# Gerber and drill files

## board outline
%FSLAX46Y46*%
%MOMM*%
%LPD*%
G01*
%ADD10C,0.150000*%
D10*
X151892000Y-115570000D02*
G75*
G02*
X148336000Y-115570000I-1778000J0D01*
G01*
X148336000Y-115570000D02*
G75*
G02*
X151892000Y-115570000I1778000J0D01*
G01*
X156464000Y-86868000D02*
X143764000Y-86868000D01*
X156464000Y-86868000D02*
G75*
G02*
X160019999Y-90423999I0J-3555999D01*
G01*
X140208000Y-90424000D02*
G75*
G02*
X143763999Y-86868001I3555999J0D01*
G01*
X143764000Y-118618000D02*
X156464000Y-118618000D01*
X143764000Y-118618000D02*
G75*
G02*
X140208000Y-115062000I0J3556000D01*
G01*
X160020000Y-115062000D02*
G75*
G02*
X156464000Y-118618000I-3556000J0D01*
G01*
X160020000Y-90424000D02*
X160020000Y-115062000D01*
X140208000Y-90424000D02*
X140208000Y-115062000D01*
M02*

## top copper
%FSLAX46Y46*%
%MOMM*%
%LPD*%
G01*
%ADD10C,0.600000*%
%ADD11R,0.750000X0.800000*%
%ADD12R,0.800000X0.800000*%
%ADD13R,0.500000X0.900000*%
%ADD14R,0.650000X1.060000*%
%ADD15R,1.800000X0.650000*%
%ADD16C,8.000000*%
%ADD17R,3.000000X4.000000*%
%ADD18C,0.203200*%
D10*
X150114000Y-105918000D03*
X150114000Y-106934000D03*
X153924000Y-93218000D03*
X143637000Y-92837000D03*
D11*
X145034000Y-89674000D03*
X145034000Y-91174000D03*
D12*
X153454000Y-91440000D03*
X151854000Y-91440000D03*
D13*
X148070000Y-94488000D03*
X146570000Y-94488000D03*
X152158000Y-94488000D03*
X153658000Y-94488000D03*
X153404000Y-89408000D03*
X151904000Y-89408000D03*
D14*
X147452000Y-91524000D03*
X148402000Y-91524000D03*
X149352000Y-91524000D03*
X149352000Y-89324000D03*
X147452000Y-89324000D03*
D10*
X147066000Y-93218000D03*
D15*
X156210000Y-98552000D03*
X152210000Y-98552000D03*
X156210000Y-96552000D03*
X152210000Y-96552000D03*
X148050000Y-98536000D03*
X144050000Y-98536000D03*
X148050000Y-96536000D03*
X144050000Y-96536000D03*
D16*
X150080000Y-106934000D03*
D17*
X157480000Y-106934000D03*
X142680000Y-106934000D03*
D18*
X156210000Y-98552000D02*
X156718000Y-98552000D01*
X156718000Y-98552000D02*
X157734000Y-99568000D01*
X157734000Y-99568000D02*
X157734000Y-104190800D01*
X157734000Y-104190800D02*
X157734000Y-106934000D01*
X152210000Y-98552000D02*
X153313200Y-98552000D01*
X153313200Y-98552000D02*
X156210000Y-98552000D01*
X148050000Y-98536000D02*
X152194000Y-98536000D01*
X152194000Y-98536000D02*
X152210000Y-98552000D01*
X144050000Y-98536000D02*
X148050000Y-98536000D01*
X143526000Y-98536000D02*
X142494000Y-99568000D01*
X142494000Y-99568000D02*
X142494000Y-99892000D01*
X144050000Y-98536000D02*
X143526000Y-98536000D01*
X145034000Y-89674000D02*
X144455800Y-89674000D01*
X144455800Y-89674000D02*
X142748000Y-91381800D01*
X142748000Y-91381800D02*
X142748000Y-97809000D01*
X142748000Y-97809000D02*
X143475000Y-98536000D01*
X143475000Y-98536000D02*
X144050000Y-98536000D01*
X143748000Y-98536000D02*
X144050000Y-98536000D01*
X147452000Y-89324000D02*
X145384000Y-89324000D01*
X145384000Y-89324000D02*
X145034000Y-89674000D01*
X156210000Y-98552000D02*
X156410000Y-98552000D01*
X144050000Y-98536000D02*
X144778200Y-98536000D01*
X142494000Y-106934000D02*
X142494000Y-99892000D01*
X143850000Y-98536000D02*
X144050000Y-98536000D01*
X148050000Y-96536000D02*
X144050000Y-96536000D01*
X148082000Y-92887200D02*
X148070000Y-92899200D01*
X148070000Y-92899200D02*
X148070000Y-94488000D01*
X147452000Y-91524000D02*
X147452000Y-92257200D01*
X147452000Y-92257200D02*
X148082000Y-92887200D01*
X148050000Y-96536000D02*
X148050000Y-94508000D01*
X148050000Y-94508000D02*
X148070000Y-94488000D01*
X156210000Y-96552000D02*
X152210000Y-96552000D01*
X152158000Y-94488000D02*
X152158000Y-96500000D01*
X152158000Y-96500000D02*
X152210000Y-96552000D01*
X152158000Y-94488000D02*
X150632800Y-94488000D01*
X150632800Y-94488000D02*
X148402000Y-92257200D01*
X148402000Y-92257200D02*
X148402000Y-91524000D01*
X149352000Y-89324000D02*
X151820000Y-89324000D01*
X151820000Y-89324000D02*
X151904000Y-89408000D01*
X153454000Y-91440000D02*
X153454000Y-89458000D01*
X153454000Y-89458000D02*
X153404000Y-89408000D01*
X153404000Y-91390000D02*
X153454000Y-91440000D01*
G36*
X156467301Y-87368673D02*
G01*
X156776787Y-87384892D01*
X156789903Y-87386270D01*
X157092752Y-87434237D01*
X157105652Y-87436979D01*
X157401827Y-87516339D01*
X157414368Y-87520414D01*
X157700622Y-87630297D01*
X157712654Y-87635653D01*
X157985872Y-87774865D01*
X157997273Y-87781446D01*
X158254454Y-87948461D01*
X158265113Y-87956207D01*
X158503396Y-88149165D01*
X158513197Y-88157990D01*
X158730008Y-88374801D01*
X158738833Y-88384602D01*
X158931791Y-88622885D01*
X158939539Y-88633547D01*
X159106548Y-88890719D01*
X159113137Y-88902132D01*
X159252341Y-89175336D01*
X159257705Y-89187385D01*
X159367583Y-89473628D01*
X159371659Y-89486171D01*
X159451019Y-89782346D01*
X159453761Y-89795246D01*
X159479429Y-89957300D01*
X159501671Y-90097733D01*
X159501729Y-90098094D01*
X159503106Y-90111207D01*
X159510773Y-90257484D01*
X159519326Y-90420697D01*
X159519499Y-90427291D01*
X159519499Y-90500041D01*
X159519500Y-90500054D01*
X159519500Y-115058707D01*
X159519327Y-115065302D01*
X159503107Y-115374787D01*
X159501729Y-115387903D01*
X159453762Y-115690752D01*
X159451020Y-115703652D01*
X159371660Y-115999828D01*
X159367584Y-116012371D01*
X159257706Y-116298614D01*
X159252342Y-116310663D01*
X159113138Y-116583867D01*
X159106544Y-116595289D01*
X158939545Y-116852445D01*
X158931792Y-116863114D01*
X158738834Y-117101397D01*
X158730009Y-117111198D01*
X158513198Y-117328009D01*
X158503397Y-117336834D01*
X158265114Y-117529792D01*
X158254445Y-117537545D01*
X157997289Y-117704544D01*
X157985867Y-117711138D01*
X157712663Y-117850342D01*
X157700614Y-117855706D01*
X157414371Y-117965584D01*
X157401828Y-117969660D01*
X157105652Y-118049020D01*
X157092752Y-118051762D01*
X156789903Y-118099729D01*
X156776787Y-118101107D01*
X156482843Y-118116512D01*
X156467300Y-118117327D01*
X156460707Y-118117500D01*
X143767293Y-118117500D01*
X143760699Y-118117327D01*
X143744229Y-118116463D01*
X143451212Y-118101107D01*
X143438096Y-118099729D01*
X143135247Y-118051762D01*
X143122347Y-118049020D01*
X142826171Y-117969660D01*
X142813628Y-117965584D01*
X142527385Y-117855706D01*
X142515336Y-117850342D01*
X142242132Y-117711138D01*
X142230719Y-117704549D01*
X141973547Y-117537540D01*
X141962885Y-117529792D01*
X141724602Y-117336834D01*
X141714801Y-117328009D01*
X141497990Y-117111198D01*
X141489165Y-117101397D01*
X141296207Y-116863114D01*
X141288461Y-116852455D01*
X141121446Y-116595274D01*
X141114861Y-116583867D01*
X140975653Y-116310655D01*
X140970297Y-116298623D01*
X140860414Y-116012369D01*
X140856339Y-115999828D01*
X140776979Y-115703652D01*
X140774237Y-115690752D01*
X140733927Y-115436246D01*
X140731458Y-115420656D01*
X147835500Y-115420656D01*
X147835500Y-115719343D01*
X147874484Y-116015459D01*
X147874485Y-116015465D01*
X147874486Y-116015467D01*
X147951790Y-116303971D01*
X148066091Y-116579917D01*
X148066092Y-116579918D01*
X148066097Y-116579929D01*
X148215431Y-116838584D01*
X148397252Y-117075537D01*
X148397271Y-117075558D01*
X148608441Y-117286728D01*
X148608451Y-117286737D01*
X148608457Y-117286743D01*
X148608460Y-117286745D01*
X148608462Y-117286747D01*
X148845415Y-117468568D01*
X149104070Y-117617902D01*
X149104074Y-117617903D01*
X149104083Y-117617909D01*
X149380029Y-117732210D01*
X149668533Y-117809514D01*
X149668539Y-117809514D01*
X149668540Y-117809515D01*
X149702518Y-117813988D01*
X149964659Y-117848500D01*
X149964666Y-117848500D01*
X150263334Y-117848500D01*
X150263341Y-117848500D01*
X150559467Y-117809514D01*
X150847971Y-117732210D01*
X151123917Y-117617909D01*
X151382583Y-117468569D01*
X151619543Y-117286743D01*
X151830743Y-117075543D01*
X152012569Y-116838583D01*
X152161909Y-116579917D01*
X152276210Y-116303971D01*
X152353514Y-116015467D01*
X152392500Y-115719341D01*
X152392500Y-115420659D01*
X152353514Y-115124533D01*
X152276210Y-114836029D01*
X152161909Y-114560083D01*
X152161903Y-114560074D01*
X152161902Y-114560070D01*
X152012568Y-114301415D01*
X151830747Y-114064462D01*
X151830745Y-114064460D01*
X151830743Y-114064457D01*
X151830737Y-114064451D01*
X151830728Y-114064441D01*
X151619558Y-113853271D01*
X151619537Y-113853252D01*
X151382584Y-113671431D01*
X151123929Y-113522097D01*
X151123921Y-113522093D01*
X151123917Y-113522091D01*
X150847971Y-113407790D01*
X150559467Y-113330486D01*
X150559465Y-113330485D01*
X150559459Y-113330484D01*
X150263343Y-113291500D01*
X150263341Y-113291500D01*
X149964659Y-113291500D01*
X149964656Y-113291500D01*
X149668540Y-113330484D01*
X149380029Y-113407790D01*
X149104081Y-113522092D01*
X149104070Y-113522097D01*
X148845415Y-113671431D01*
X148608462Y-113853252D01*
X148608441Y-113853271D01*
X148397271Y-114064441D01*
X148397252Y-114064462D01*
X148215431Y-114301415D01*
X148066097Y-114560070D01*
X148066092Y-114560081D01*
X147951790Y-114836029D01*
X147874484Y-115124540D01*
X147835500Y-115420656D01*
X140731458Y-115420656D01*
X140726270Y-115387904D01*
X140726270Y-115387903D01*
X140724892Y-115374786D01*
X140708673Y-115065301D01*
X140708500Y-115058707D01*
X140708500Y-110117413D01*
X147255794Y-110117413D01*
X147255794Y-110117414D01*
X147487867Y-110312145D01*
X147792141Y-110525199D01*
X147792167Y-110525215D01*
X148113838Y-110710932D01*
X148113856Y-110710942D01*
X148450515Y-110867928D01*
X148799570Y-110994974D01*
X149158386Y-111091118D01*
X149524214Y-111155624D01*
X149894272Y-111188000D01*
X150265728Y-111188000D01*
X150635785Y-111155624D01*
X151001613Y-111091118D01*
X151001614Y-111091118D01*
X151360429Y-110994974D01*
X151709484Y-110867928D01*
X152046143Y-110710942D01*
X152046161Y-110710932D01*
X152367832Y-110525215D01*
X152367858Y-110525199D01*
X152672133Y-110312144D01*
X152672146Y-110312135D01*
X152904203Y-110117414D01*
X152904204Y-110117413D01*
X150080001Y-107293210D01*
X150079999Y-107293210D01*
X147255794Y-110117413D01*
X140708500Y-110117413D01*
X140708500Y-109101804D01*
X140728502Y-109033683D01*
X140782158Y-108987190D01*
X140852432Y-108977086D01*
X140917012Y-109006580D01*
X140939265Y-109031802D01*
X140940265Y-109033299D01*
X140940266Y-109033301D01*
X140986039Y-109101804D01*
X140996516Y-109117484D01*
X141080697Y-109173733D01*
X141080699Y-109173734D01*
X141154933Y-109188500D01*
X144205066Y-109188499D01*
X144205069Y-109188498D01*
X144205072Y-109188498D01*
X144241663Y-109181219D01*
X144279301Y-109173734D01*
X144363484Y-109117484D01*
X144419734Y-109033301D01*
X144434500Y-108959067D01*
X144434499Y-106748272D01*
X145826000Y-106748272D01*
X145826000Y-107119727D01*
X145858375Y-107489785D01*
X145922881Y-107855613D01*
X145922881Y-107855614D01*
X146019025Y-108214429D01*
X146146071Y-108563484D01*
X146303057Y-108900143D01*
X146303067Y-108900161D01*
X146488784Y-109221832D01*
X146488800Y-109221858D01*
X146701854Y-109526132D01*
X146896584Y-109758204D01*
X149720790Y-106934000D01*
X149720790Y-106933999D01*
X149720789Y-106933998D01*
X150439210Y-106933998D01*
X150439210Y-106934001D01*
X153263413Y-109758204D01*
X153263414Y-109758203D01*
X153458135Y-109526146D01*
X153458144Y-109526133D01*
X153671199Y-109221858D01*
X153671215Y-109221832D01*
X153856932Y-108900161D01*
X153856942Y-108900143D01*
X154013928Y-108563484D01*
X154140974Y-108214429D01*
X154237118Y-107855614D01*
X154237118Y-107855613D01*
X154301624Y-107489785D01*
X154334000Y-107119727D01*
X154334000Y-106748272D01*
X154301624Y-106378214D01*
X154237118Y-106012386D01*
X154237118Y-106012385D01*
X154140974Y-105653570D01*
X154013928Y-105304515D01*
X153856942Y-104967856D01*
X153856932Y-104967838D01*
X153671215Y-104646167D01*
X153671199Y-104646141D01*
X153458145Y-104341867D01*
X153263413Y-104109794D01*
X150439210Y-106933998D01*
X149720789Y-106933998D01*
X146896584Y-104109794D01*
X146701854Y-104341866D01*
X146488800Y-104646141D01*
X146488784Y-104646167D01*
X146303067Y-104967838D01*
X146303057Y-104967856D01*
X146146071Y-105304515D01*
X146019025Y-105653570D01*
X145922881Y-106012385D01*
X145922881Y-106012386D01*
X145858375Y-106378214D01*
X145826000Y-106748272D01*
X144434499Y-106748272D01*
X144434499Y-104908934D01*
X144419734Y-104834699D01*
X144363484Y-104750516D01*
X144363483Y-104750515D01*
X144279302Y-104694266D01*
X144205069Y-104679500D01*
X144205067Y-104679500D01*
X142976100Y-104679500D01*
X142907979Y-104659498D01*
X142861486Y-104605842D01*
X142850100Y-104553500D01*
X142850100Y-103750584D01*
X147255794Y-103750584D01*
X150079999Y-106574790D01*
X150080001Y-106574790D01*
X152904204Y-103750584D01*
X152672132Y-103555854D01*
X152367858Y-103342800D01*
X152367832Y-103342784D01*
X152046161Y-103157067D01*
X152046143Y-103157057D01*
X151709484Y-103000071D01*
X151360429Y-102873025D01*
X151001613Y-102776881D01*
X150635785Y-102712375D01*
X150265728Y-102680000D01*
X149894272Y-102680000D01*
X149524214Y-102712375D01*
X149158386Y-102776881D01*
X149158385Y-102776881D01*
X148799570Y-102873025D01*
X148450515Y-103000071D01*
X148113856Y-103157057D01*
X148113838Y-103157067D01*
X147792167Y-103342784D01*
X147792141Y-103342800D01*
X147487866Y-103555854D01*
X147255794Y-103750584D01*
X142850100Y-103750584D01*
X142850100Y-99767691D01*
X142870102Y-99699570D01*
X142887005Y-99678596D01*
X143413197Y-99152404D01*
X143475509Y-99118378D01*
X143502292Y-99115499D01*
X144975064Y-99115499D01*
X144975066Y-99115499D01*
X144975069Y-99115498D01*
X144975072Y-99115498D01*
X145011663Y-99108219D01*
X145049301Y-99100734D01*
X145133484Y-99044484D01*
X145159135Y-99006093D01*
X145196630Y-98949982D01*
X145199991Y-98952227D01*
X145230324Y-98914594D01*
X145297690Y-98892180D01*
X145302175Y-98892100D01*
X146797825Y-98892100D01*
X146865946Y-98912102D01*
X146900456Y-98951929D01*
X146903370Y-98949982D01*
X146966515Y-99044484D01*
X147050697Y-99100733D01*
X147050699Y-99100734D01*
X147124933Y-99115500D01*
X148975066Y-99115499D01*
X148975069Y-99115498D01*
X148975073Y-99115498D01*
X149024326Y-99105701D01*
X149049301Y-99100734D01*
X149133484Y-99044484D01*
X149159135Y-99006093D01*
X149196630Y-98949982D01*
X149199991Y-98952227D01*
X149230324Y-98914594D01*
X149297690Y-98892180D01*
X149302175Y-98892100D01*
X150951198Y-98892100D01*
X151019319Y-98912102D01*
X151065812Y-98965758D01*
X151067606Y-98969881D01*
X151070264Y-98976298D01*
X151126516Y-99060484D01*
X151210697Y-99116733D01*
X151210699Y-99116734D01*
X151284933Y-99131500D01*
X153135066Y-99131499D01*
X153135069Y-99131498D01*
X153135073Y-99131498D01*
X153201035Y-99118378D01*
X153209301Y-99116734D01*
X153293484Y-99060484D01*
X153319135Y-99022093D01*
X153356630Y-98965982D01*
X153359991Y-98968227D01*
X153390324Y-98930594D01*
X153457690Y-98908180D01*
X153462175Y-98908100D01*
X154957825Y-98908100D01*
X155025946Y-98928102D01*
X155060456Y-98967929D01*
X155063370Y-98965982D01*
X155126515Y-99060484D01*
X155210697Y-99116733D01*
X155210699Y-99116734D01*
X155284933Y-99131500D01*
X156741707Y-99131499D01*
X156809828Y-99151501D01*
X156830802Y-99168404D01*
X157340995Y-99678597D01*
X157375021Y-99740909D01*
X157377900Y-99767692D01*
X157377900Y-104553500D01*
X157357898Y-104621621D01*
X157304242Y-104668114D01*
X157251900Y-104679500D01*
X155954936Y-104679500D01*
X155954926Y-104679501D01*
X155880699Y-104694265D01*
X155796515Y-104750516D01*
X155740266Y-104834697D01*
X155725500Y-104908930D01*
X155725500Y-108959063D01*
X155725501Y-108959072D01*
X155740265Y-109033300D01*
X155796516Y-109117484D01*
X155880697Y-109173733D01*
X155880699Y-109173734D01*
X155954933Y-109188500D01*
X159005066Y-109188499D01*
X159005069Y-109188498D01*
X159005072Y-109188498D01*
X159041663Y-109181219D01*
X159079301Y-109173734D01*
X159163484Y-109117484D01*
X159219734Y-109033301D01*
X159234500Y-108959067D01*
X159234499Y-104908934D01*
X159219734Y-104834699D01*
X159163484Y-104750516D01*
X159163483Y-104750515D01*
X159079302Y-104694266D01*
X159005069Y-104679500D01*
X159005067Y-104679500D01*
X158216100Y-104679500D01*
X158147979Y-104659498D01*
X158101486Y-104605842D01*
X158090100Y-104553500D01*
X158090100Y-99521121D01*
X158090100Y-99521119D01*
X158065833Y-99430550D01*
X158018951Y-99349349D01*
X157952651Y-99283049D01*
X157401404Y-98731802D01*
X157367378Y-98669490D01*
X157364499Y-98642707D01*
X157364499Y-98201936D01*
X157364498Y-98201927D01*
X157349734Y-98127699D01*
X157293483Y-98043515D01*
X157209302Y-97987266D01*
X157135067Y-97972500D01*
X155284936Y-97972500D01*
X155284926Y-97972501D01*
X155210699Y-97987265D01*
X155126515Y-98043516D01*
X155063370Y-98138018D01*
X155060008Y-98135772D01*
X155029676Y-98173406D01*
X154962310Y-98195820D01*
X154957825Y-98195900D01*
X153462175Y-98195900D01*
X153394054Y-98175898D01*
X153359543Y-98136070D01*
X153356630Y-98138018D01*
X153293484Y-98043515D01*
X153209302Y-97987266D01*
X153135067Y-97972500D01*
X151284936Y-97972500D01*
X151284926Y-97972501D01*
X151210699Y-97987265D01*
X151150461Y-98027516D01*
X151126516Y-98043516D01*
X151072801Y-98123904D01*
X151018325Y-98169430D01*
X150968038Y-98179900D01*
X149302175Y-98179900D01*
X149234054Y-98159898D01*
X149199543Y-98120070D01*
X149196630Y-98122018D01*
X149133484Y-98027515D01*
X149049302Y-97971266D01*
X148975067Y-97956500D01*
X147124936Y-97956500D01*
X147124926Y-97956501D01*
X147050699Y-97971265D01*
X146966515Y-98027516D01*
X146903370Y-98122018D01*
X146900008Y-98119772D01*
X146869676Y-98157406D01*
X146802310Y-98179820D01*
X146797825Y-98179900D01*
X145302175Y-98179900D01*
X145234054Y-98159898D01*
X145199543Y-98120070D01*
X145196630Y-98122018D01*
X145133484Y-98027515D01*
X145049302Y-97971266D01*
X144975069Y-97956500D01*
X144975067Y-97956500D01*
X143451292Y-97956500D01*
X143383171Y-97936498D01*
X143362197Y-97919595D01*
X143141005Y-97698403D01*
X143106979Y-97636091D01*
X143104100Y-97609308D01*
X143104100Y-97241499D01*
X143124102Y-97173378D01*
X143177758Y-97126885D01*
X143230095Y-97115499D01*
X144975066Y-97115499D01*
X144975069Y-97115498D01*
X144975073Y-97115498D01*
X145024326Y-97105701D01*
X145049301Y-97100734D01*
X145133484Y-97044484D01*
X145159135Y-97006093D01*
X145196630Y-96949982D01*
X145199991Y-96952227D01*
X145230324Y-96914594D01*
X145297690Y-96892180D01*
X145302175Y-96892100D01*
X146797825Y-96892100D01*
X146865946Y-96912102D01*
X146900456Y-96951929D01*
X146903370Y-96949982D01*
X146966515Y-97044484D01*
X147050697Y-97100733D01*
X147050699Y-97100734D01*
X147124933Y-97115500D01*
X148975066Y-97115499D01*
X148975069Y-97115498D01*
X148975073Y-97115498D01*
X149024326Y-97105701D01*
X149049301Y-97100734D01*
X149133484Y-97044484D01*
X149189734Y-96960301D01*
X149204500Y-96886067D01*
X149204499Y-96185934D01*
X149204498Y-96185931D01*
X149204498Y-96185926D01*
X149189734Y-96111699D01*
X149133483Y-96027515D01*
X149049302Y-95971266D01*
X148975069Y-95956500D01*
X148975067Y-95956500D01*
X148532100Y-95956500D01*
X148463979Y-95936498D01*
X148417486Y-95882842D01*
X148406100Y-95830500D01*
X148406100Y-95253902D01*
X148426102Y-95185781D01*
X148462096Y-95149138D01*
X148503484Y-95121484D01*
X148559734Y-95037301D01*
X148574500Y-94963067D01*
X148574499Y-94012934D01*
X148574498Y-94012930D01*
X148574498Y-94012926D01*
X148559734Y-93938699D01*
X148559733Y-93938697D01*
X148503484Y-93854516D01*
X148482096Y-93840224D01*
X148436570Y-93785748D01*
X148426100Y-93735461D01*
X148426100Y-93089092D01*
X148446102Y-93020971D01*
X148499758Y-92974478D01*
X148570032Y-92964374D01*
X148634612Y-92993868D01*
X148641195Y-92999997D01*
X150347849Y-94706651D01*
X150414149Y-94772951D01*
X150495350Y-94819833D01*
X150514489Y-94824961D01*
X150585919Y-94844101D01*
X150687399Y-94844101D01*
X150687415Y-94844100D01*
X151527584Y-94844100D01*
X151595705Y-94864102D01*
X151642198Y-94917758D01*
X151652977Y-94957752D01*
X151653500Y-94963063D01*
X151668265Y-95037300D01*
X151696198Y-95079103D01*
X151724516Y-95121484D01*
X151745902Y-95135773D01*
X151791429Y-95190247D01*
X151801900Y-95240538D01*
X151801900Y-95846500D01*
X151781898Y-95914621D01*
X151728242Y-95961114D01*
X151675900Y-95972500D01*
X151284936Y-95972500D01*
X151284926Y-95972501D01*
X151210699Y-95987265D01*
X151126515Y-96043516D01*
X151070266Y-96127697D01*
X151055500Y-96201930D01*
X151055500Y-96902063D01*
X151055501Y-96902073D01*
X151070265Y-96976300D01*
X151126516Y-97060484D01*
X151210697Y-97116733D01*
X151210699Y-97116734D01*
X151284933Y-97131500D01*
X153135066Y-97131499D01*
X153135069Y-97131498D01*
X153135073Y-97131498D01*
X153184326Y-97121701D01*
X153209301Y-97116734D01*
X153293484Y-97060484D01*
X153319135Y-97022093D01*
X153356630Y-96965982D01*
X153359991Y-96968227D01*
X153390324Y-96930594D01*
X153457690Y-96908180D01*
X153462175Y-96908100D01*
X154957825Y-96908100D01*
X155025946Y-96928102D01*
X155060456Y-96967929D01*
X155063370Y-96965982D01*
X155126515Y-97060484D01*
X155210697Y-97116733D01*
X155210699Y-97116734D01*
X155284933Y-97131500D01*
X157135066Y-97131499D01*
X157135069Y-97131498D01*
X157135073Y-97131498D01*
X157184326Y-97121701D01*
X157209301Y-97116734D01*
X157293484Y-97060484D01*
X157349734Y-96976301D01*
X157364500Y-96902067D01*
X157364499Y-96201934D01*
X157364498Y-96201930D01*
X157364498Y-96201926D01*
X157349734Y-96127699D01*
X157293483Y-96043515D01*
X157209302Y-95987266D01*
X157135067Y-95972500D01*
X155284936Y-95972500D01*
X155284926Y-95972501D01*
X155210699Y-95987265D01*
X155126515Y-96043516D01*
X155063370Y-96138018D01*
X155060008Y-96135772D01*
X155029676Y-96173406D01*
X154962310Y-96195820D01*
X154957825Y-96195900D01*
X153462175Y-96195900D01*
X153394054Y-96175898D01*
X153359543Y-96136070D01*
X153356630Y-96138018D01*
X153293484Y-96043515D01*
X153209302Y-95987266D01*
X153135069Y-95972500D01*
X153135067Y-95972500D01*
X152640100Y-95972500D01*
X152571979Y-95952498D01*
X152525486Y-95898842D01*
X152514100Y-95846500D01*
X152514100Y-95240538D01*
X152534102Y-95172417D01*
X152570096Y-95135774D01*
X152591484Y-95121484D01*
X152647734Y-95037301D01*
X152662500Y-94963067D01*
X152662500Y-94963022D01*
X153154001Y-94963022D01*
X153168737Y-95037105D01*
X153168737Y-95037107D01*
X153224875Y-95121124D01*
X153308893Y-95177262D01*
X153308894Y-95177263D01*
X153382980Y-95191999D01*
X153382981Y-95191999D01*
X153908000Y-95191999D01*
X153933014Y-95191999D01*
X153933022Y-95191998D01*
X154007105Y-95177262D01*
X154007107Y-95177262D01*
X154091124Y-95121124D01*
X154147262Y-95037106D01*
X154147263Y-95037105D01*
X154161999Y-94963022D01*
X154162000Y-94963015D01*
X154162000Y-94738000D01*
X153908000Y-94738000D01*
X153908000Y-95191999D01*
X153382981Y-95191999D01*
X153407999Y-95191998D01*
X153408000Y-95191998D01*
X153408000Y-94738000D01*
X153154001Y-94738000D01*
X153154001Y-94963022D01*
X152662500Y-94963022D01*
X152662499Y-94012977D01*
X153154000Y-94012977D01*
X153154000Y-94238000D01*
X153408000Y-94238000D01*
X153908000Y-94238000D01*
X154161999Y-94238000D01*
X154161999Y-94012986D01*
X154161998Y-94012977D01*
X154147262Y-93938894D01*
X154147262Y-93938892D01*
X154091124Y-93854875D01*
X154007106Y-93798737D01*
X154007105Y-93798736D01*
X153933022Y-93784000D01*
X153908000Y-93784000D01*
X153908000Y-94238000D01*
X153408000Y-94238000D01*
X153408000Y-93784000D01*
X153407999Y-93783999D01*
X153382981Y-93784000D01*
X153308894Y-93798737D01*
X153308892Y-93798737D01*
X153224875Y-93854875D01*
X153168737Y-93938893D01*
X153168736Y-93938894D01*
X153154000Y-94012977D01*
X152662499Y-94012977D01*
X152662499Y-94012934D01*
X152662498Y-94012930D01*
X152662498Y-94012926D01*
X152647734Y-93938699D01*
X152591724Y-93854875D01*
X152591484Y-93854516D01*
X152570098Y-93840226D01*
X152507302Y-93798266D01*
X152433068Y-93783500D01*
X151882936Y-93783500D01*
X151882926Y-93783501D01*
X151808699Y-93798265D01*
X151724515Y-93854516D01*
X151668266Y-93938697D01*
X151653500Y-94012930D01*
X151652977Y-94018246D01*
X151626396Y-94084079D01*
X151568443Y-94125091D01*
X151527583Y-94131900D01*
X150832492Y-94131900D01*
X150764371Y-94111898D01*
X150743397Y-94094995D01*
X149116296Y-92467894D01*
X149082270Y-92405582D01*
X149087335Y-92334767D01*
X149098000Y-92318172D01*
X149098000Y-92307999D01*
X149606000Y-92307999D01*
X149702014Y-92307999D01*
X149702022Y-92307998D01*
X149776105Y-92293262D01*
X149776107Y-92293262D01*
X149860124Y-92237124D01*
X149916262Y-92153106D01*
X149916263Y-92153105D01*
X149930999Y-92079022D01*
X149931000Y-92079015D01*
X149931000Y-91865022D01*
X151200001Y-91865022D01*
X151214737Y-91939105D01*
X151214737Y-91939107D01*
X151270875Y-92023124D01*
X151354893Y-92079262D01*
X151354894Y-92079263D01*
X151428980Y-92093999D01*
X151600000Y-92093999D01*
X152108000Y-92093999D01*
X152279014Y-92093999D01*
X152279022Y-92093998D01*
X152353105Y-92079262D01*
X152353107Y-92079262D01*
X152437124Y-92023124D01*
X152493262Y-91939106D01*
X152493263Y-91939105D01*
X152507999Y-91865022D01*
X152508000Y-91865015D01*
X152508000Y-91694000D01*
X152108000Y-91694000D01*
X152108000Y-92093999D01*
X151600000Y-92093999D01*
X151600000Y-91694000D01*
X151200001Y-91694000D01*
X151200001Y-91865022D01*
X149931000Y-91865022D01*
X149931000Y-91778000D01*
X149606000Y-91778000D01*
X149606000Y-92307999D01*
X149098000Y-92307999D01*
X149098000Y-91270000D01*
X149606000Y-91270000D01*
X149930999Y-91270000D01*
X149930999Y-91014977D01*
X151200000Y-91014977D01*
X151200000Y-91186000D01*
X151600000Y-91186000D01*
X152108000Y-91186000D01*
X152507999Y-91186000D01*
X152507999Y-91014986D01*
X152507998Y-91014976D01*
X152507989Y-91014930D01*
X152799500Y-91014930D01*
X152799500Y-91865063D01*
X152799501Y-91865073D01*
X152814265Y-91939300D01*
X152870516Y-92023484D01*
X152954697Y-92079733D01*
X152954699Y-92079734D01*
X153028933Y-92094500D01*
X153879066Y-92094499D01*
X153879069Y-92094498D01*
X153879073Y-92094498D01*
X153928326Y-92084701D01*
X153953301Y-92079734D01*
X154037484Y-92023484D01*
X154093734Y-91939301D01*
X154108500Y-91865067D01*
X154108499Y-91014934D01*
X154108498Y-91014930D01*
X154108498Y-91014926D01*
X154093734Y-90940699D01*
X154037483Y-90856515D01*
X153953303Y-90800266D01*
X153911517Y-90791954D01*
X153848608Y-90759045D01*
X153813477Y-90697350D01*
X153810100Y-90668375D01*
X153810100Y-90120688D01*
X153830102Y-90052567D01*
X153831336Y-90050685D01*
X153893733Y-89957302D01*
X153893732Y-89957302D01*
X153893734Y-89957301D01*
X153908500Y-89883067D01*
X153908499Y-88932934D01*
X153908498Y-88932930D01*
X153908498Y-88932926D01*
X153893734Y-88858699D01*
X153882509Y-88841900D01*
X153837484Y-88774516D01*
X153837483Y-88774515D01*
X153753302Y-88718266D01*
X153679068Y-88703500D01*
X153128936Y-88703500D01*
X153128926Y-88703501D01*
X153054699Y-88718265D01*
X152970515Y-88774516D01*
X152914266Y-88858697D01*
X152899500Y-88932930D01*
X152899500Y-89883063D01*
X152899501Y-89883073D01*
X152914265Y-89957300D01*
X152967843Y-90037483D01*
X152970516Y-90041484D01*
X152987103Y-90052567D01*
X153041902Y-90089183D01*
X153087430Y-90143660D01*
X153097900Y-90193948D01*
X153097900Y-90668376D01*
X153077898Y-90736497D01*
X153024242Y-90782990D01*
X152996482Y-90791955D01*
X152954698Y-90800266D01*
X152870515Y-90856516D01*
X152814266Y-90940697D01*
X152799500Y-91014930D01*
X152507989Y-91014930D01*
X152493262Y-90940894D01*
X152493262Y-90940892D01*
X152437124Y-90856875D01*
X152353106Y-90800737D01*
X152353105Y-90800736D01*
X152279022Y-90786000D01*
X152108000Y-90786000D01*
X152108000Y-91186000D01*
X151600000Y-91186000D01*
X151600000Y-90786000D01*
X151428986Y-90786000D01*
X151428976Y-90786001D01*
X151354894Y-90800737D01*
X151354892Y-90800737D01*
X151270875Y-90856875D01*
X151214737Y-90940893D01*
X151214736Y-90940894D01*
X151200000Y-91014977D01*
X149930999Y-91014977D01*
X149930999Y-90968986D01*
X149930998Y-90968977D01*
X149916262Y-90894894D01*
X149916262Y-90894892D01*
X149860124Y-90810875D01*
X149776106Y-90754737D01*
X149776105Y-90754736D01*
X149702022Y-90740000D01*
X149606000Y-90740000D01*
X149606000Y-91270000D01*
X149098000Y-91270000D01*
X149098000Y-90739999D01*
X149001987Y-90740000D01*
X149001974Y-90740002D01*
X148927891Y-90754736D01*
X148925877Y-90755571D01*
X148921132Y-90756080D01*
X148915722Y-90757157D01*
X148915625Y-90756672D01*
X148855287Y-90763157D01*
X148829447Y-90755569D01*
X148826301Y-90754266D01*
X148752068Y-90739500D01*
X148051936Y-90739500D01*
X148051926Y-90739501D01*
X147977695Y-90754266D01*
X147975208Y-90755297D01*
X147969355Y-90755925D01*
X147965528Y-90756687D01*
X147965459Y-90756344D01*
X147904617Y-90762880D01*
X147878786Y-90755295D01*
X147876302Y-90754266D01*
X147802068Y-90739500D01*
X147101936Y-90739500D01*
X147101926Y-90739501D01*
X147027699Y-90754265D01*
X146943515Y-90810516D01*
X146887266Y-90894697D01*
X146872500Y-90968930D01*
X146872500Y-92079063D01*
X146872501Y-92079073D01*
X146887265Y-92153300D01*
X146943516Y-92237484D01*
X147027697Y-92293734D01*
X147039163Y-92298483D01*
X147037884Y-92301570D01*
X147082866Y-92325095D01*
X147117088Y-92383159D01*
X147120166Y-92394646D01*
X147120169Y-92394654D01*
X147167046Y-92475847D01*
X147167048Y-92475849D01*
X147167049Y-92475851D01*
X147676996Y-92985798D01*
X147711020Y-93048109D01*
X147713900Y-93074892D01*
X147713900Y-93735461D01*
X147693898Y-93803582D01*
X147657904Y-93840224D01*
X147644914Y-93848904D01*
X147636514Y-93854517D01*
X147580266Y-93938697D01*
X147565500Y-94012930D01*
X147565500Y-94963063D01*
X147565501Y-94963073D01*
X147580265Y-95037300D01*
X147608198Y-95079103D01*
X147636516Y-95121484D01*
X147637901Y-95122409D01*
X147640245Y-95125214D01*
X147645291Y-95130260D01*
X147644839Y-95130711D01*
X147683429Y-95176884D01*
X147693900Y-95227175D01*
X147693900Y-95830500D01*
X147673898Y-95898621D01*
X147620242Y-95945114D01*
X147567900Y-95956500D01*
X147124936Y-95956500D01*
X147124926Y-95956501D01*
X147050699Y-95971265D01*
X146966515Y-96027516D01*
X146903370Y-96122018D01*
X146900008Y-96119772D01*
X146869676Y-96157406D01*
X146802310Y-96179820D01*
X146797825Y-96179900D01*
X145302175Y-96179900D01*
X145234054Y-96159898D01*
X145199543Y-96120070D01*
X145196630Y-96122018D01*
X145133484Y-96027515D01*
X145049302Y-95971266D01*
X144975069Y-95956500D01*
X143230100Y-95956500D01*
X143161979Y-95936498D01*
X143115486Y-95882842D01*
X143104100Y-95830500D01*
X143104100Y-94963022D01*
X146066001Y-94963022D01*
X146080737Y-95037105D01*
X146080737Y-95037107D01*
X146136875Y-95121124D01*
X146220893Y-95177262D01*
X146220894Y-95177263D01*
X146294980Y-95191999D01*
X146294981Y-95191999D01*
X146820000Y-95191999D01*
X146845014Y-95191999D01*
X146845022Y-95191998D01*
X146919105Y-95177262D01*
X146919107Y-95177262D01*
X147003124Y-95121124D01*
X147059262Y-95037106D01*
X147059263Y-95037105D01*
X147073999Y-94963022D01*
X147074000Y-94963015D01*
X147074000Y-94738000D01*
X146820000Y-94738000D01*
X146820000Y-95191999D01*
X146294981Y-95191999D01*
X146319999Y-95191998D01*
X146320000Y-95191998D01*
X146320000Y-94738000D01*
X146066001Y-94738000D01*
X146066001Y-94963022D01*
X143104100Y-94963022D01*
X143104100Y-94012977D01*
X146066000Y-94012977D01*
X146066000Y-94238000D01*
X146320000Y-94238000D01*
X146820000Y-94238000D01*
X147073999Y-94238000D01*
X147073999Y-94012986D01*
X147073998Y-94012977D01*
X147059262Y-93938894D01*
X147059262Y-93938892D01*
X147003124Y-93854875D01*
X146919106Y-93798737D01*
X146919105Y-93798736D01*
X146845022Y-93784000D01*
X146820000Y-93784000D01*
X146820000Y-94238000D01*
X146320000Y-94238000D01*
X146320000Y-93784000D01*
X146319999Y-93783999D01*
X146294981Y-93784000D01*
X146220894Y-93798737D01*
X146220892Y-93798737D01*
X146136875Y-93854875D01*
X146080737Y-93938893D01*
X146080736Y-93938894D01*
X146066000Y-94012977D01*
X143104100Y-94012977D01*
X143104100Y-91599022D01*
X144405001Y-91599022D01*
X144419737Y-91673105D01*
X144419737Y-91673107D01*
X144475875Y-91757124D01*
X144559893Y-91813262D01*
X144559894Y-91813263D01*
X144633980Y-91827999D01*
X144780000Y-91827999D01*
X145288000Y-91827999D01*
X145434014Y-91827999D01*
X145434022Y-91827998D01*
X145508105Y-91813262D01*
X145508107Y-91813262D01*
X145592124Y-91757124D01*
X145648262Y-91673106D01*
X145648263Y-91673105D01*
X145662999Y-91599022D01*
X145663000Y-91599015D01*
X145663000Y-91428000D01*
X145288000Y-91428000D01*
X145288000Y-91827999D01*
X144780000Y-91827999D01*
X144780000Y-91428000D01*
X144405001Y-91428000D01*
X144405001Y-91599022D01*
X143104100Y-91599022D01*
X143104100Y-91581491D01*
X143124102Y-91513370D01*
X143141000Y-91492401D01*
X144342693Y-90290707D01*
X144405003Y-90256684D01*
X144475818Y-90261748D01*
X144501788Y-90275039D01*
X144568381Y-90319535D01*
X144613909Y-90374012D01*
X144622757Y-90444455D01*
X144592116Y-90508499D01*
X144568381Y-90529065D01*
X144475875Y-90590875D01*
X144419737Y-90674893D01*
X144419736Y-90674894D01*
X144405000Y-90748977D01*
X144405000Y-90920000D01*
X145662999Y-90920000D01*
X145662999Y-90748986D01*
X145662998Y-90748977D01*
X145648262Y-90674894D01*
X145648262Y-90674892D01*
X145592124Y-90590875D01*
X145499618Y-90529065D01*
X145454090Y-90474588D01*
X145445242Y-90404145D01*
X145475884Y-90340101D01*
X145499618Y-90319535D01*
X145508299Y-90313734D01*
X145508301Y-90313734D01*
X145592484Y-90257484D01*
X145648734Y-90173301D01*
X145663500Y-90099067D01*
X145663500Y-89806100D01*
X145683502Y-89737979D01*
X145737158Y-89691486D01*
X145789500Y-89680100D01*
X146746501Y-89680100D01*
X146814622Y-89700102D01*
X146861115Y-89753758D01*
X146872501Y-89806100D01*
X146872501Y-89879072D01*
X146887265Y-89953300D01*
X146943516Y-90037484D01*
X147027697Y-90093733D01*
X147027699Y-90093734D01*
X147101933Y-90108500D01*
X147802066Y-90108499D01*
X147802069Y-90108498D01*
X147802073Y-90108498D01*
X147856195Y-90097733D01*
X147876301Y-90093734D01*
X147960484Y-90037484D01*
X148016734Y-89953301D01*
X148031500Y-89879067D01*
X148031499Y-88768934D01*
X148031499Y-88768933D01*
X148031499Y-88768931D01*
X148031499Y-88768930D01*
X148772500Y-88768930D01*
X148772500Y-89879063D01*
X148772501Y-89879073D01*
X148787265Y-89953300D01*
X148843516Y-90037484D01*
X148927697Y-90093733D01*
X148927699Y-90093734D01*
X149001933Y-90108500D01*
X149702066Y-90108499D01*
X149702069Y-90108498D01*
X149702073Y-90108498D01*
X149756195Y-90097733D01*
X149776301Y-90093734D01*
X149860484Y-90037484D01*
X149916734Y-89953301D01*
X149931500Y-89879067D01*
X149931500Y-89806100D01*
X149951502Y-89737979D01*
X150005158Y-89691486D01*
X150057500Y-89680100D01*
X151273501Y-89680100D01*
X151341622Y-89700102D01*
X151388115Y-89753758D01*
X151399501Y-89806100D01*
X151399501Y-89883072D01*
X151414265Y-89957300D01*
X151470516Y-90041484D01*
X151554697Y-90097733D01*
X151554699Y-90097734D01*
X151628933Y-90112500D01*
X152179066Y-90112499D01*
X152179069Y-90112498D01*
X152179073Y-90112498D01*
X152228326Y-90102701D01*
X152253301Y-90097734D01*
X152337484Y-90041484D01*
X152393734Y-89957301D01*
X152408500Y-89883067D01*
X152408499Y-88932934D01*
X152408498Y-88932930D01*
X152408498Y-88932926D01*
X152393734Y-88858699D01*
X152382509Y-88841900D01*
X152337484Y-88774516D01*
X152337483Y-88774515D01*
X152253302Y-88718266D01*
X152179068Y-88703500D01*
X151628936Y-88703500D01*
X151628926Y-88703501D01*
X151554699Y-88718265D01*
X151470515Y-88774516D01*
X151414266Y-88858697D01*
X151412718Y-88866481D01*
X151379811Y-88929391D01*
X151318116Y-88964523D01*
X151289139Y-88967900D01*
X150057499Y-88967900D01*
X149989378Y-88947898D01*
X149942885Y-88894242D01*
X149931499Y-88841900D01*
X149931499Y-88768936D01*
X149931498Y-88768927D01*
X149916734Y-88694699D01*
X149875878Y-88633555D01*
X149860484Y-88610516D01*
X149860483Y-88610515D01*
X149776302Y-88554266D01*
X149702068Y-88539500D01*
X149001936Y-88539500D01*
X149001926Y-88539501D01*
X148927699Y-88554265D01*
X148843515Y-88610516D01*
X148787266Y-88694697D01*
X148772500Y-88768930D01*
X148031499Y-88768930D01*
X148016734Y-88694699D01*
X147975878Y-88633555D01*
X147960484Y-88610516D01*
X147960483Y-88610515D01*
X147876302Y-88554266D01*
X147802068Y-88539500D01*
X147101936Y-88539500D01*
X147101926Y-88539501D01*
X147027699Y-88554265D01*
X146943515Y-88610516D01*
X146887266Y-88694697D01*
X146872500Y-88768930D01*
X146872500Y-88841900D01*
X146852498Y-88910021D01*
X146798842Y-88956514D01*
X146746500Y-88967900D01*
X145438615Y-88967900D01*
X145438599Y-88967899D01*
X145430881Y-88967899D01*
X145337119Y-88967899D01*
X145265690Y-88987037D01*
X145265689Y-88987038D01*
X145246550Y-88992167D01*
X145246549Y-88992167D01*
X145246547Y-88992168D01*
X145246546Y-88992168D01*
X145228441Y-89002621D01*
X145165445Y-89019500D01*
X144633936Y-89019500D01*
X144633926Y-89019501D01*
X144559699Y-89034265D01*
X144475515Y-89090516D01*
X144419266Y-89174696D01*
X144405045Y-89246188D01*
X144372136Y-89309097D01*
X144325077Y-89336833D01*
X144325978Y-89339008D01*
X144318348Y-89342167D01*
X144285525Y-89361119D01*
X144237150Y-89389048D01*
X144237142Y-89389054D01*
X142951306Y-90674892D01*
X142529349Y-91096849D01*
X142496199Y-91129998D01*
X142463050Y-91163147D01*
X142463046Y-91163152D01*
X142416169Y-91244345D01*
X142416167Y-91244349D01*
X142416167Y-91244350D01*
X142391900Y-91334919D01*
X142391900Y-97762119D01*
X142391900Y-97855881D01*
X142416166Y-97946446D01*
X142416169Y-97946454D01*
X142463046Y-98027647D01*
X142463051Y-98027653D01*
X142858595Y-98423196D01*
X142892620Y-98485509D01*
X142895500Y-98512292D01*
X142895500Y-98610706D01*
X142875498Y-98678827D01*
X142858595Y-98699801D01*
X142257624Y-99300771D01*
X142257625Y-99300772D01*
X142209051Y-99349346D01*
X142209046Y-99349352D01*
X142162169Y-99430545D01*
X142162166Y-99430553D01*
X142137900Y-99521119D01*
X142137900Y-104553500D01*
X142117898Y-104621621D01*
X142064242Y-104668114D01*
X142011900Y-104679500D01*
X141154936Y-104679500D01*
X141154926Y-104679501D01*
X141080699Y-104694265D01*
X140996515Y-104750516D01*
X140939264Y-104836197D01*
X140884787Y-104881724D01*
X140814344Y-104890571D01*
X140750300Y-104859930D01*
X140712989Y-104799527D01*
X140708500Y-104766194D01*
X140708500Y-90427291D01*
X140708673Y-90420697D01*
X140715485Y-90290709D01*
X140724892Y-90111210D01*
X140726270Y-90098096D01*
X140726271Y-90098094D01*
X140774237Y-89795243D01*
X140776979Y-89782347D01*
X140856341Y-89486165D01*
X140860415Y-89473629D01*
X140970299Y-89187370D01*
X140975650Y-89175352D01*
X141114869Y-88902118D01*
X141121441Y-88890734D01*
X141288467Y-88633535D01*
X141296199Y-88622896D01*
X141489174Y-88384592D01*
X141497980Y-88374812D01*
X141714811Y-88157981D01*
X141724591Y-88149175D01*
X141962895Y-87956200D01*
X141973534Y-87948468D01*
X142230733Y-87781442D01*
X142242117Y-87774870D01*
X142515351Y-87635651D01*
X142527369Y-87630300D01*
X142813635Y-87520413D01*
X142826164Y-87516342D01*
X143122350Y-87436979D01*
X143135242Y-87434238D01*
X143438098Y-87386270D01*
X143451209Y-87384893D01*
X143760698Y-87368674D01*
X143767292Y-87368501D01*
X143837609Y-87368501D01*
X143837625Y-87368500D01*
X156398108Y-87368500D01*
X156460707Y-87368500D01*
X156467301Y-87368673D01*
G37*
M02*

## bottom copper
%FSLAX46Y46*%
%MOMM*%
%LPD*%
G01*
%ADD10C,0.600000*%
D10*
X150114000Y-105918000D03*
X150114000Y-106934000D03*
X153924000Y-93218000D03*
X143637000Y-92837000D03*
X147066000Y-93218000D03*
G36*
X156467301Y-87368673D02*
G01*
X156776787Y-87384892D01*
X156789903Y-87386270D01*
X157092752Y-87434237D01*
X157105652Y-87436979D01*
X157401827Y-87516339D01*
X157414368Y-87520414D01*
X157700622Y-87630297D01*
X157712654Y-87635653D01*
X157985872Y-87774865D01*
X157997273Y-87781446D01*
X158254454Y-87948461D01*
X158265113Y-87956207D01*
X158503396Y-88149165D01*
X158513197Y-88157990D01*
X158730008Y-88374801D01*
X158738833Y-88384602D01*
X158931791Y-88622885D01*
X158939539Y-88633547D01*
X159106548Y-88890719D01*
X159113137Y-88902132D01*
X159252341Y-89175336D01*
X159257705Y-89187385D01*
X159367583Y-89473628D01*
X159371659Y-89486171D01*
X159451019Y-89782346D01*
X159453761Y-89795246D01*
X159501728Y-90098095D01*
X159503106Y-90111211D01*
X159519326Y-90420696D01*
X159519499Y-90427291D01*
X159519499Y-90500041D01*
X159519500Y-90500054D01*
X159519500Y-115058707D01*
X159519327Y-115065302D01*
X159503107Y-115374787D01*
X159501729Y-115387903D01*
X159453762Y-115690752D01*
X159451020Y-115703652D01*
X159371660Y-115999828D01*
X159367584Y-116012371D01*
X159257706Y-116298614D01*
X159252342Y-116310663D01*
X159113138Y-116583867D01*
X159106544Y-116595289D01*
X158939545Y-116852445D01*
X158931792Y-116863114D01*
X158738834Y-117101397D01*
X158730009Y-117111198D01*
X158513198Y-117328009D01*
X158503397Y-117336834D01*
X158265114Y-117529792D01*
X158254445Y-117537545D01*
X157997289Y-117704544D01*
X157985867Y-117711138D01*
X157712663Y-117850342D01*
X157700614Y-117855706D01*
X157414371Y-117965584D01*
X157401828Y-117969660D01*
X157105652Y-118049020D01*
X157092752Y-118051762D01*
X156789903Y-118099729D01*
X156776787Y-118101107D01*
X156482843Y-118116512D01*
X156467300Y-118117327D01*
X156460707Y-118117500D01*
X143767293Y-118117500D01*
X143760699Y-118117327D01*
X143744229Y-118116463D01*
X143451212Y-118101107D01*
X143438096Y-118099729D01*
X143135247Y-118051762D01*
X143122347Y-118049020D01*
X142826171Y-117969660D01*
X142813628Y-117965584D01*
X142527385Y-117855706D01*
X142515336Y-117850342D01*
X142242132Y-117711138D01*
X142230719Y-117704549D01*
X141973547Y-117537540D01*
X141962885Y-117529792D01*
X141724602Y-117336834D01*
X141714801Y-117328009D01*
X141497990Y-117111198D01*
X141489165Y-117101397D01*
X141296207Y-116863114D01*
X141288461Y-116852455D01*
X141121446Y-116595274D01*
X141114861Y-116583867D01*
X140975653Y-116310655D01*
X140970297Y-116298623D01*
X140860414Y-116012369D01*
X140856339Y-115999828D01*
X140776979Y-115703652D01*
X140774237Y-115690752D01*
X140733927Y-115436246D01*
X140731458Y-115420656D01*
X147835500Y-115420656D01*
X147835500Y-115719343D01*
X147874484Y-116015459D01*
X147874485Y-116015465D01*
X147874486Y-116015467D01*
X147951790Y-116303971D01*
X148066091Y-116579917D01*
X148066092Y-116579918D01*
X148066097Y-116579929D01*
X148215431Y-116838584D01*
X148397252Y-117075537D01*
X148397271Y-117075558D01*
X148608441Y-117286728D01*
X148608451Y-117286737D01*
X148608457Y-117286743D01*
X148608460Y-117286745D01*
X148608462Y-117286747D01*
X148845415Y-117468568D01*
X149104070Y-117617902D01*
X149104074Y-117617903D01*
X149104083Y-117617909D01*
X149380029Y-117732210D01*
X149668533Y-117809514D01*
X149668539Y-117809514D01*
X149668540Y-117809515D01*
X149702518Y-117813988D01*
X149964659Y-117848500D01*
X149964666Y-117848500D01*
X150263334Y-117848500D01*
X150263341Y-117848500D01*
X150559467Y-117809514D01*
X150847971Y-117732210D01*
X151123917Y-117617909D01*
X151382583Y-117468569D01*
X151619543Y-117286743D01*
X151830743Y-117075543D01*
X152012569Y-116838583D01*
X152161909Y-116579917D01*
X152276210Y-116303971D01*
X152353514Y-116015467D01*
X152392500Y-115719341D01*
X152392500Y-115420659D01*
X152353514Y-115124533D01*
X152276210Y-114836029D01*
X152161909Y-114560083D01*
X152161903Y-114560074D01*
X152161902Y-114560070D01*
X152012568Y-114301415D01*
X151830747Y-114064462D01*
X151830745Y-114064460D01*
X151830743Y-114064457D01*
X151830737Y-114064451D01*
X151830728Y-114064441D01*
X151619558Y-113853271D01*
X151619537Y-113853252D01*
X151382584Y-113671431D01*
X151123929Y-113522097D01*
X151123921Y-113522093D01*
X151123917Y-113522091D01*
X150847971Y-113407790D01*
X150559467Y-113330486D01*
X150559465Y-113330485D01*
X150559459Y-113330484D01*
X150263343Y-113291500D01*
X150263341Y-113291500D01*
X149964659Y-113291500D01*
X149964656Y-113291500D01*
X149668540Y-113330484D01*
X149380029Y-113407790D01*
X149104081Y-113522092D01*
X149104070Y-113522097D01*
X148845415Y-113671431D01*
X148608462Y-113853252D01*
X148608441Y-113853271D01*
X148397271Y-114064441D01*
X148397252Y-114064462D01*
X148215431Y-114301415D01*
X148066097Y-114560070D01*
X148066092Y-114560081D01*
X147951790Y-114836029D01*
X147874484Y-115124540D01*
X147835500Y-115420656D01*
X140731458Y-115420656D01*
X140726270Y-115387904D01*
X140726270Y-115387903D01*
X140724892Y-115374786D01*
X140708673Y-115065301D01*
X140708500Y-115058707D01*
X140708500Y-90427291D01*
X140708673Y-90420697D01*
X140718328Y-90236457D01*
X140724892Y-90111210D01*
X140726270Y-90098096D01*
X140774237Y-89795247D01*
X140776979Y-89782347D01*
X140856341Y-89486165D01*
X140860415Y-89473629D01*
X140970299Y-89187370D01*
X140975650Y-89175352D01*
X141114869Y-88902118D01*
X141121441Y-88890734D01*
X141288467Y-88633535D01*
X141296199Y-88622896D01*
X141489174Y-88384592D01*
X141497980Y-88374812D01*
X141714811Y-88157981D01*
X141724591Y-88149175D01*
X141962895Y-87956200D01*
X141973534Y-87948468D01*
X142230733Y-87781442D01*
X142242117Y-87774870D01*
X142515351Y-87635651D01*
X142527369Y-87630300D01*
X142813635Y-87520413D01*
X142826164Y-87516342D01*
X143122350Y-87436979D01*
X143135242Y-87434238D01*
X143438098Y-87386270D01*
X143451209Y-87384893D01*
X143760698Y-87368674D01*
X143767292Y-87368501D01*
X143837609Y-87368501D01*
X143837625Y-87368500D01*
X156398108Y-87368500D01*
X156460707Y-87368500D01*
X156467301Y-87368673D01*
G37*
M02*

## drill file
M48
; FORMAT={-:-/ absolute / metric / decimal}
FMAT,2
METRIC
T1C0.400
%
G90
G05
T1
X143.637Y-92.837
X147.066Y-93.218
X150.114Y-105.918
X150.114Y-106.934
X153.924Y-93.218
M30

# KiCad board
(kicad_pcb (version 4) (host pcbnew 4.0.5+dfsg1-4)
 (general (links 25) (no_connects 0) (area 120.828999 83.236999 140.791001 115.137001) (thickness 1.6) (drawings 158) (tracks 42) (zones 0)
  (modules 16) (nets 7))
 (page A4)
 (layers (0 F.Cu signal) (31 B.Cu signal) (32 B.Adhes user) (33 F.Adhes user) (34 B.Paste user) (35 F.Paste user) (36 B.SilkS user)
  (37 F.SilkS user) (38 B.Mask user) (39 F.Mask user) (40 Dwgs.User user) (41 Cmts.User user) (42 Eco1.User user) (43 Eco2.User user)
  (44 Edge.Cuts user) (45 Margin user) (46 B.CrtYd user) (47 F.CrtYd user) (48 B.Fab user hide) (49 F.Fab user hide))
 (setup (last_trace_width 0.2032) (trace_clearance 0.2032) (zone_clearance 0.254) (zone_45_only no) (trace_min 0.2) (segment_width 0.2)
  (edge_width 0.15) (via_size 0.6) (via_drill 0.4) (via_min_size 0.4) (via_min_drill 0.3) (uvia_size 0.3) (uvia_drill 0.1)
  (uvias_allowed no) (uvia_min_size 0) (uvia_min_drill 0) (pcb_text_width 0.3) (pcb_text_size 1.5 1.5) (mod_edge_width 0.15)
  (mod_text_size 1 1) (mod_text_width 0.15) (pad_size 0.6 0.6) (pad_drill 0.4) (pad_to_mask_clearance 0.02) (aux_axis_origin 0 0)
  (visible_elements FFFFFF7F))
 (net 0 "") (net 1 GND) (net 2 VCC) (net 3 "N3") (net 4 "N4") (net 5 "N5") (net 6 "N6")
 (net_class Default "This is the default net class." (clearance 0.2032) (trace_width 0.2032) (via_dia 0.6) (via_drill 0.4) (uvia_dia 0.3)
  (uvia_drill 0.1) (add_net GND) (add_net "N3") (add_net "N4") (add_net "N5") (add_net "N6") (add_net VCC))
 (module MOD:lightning (layer F.Cu) (at 142.24 89.662 90)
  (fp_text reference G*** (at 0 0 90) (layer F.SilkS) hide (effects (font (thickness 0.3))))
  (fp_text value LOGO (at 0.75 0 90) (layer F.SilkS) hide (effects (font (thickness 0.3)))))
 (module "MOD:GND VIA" (layer F.Cu) (at 150.114 104.648)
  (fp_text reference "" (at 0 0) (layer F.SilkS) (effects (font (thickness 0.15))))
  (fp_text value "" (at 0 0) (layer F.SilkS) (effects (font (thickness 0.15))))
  (pad 1 thru_hole circle (at 0 1.27) (size 0.6 0.6) (drill 0.4) (layers *.Cu) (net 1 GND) (zone_connect 2)))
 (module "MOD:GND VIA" (layer F.Cu) (at 150.114 105.664)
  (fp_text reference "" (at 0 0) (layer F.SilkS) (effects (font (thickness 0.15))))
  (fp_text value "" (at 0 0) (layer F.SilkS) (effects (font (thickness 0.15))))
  (pad 1 thru_hole circle (at 0 1.27) (size 0.6 0.6) (drill 0.4) (layers *.Cu) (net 1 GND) (zone_connect 2)))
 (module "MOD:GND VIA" (layer F.Cu) (at 153.924 91.948)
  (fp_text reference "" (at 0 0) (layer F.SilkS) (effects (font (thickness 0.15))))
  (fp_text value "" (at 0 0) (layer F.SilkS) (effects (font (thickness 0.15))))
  (pad 1 thru_hole circle (at 0 1.27) (size 0.6 0.6) (drill 0.4) (layers *.Cu) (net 1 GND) (zone_connect 2)))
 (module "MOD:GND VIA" (layer F.Cu) (at 143.637 91.567)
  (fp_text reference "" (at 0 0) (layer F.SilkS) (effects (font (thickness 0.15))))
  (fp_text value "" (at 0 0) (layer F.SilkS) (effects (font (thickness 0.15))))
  (pad 1 thru_hole circle (at 0 1.27) (size 0.6 0.6) (drill 0.4) (layers *.Cu) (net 1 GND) (zone_connect 2)))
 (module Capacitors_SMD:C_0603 (layer F.Cu) (at 145.034 90.424 90)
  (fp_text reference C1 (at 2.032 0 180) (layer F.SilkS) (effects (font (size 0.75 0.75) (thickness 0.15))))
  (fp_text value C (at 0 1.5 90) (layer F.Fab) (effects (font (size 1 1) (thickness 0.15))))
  (pad 2 smd rect (at 0.75 0 90) (size 0.8 0.75) (layers F.Cu F.Paste F.Mask) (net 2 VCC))
  (pad 1 smd rect (at -0.75 0 90) (size 0.8 0.75) (layers F.Cu F.Paste F.Mask) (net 1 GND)))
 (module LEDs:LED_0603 (layer F.Cu) (at 152.654 91.44)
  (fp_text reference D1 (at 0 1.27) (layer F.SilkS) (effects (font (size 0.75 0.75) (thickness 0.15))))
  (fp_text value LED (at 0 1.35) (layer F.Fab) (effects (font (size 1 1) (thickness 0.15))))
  (pad 2 smd rect (at 0.8 0 180) (size 0.8 0.8) (layers F.Cu F.Paste F.Mask) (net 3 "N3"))
  (pad 1 smd rect (at -0.8 0 180) (size 0.8 0.8) (layers F.Cu F.Paste F.Mask) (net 1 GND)))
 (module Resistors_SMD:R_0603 (layer F.Cu) (at 147.32 94.488 180)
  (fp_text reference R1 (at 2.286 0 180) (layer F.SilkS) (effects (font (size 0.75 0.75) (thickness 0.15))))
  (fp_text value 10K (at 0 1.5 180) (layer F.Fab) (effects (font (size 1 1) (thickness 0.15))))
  (pad 1 smd rect (at -0.75 0 180) (size 0.5 0.9) (layers F.Cu F.Paste F.Mask) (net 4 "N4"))
  (pad 2 smd rect (at 0.75 0 180) (size 0.5 0.9) (layers F.Cu F.Paste F.Mask) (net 1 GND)))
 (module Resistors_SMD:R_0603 (layer F.Cu) (at 152.908 94.488)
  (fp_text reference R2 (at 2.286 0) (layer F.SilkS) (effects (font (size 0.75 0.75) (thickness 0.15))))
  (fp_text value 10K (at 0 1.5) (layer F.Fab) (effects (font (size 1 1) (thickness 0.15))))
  (pad 1 smd rect (at -0.75 0) (size 0.5 0.9) (layers F.Cu F.Paste F.Mask) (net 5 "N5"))
  (pad 2 smd rect (at 0.75 0) (size 0.5 0.9) (layers F.Cu F.Paste F.Mask) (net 1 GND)))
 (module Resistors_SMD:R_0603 (layer F.Cu) (at 152.654 89.408 180)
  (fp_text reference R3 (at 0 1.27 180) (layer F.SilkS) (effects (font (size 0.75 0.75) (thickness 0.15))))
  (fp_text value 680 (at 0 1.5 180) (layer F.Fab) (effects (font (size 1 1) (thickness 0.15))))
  (pad 1 smd rect (at -0.75 0 180) (size 0.5 0.9) (layers F.Cu F.Paste F.Mask) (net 3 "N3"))
  (pad 2 smd rect (at 0.75 0 180) (size 0.5 0.9) (layers F.Cu F.Paste F.Mask) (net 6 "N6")))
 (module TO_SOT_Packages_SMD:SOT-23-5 (layer F.Cu) (at 148.402 90.424 90)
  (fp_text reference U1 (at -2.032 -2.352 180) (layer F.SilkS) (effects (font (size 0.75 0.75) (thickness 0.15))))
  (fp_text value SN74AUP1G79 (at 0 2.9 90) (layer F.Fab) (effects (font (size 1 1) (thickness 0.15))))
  (pad 1 smd rect (at -1.1 -0.95 90) (size 1.06 0.65) (layers F.Cu F.Paste F.Mask) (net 4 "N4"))
  (pad 2 smd rect (at -1.1 0 90) (size 1.06 0.65) (layers F.Cu F.Paste F.Mask) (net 5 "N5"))
  (pad 3 smd rect (at -1.1 0.95 90) (size 1.06 0.65) (layers F.Cu F.Paste F.Mask) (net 1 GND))
  (pad 4 smd rect (at 1.1 0.95 90) (size 1.06 0.65) (layers F.Cu F.Paste F.Mask) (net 6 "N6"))
  (pad 5 smd rect (at 1.1 -0.95 90) (size 1.06 0.65) (layers F.Cu F.Paste F.Mask) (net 2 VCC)))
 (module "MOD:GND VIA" (layer F.Cu) (at 147.066 91.948)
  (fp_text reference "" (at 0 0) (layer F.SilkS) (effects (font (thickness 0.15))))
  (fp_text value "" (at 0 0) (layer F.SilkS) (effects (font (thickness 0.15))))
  (pad 1 thru_hole circle (at 0 1.27) (size 0.6 0.6) (drill 0.4) (layers *.Cu) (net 1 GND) (zone_connect 2)))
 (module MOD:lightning (layer B.Cu) (at 157.48 90.424 270)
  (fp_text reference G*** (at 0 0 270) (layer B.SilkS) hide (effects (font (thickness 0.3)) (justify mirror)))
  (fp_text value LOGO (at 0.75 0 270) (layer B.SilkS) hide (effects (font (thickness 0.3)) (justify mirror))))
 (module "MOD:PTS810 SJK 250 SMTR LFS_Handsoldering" (layer F.Cu) (at 154.21 97.552 180)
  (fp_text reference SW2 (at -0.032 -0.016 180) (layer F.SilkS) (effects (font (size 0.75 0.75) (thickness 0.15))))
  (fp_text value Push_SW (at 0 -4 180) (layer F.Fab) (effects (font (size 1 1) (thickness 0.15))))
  (pad 1 smd rect (at -2 -1 180) (size 1.8 0.65) (layers F.Cu F.Paste F.Mask) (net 2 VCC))
  (pad 1 smd rect (at 2 -1 180) (size 1.8 0.65) (layers F.Cu F.Paste F.Mask) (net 2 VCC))
  (pad 2 smd rect (at -2 1 180) (size 1.8 0.65) (layers F.Cu F.Paste F.Mask) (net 5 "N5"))
  (pad 2 smd rect (at 2 1 180) (size 1.8 0.65) (layers F.Cu F.Paste F.Mask) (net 5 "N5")))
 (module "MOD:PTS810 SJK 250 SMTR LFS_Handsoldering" (layer F.Cu) (at 146.05 97.536 180)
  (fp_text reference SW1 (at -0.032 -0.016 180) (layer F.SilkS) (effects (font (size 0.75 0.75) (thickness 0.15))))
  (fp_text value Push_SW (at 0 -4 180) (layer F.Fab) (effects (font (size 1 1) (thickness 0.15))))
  (pad 1 smd rect (at -2 -1 180) (size 1.8 0.65) (layers F.Cu F.Paste F.Mask) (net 2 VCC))
  (pad 1 smd rect (at 2 -1 180) (size 1.8 0.65) (layers F.Cu F.Paste F.Mask) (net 2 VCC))
  (pad 2 smd rect (at -2 1 180) (size 1.8 0.65) (layers F.Cu F.Paste F.Mask) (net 4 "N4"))
  (pad 2 smd rect (at 2 1 180) (size 1.8 0.65) (layers F.Cu F.Paste F.Mask) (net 4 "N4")))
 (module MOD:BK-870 (layer F.Cu) (at 150.08 107.034 180)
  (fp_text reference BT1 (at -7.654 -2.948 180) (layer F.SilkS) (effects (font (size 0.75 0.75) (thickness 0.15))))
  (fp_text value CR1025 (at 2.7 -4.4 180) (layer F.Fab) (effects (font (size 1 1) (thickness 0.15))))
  (pad 2 smd circle (at 0 0.1 180) (size 8 8) (layers F.Cu F.Mask) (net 1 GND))
  (pad 1 smd rect (at -7.4 0.1 180) (size 3 4) (layers F.Cu F.Mask) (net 2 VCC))
  (pad 1 smd rect (at 7.4 0.1 180) (size 3 4) (layers F.Cu F.Mask) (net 2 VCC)))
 (gr_circle (center 150.114 115.57) (end 151.892 115.57) (layer Edge.Cuts) (width 0.15))
 (gr_line (start 156.464 86.868) (end 143.764 86.868) (layer Edge.Cuts) (width 0.15))
 (gr_arc (start 156.464 90.423999) (end 156.464 86.868) (angle 90) (layer Edge.Cuts) (width 0.15))
 (gr_arc (start 143.763999 90.424) (end 140.208 90.424) (angle 90) (layer Edge.Cuts) (width 0.15))
 (gr_line (start 143.764 118.618) (end 156.464 118.618) (layer Edge.Cuts) (width 0.15))
 (gr_arc (start 143.764 115.062) (end 143.764 118.618) (angle 90) (layer Edge.Cuts) (width 0.15))
 (gr_arc (start 156.464 115.062) (end 160.02 115.062) (angle 90) (layer Edge.Cuts) (width 0.15))
 (gr_line (start 160.02 90.424) (end 160.02 115.062) (layer Edge.Cuts) (width 0.15))
 (gr_line (start 140.208 90.424) (end 140.208 115.062) (layer Edge.Cuts) (width 0.15))
 (segment (start 156.21 98.552) (end 156.718 98.552) (width 0.2032) (layer F.Cu) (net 2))
 (segment (start 156.718 98.552) (end 157.734 99.568) (width 0.2032) (layer F.Cu) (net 2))
 (segment (start 157.734 99.568) (end 157.734 104.1908) (width 0.2032) (layer F.Cu) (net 2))
 (segment (start 157.734 104.1908) (end 157.734 106.934) (width 0.2032) (layer F.Cu) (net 2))
 (segment (start 152.21 98.552) (end 153.3132 98.552) (width 0.2032) (layer F.Cu) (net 2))
 (segment (start 153.3132 98.552) (end 156.21 98.552) (width 0.2032) (layer F.Cu) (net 2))
 (segment (start 148.05 98.536) (end 152.194 98.536) (width 0.2032) (layer F.Cu) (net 2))
 (segment (start 152.194 98.536) (end 152.21 98.552) (width 0.2032) (layer F.Cu) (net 2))
 (segment (start 144.05 98.536) (end 148.05 98.536) (width 0.2032) (layer F.Cu) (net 2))
 (segment (start 143.526 98.536) (end 142.494 99.568) (width 0.2032) (layer F.Cu) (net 2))
 (segment (start 142.494 99.568) (end 142.494 99.892) (width 0.2032) (layer F.Cu) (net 2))
 (segment (start 144.05 98.536) (end 143.526 98.536) (width 0.2032) (layer F.Cu) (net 2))
 (segment (start 145.034 89.674) (end 144.4558 89.674) (width 0.2032) (layer F.Cu) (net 2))
 (segment (start 144.4558 89.674) (end 142.748 91.3818) (width 0.2032) (layer F.Cu) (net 2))
 (segment (start 142.748 91.3818) (end 142.748 97.809) (width 0.2032) (layer F.Cu) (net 2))
 (segment (start 142.748 97.809) (end 143.475 98.536) (width 0.2032) (layer F.Cu) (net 2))
 (segment (start 143.475 98.536) (end 144.05 98.536) (width 0.2032) (layer F.Cu) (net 2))
 (segment (start 143.748 98.536) (end 144.05 98.536) (width 0.2032) (layer F.Cu) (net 2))
 (segment (start 147.452 89.324) (end 145.384 89.324) (width 0.2032) (layer F.Cu) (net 2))
 (segment (start 145.384 89.324) (end 145.034 89.674) (width 0.2032) (layer F.Cu) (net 2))
 (segment (start 156.21 98.552) (end 156.41 98.552) (width 0.2032) (layer F.Cu) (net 2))
 (segment (start 144.05 98.536) (end 144.7782 98.536) (width 0.2032) (layer F.Cu) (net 2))
 (segment (start 142.494 106.934) (end 142.494 99.892) (width 0.2032) (layer F.Cu) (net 2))
 (segment (start 143.85 98.536) (end 144.05 98.536) (width 0.2032) (layer F.Cu) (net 2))
 (segment (start 148.05 96.536) (end 144.05 96.536) (width 0.2032) (layer F.Cu) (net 4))
 (segment (start 148.082 92.8872) (end 148.07 92.8992) (width 0.2032) (layer F.Cu) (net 4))
 (segment (start 148.07 92.8992) (end 148.07 94.488) (width 0.2032) (layer F.Cu) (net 4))
 (segment (start 147.452 91.524) (end 147.452 92.2572) (width 0.2032) (layer F.Cu) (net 4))
 (segment (start 147.452 92.2572) (end 148.082 92.8872) (width 0.2032) (layer F.Cu) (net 4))
 (segment (start 148.05 96.536) (end 148.05 94.508) (width 0.2032) (layer F.Cu) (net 4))
 (segment (start 148.05 94.508) (end 148.07 94.488) (width 0.2032) (layer F.Cu) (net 4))
 (segment (start 156.21 96.552) (end 152.21 96.552) (width 0.2032) (layer F.Cu) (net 5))
 (segment (start 152.158 94.488) (end 152.158 96.5) (width 0.2032) (layer F.Cu) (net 5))
 (segment (start 152.158 96.5) (end 152.21 96.552) (width 0.2032) (layer F.Cu) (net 5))
 (segment (start 152.158 94.488) (end 150.6328 94.488) (width 0.2032) (layer F.Cu) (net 5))
 (segment (start 150.6328 94.488) (end 148.402 92.2572) (width 0.2032) (layer F.Cu) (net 5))
 (segment (start 148.402 92.2572) (end 148.402 91.524) (width 0.2032) (layer F.Cu) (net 5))
 (segment (start 149.352 89.324) (end 151.82 89.324) (width 0.2032) (layer F.Cu) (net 6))
 (segment (start 151.82 89.324) (end 151.904 89.408) (width 0.2032) (layer F.Cu) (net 6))
 (segment (start 153.454 91.44) (end 153.454 89.458) (width 0.2032) (layer F.Cu) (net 3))
 (segment (start 153.454 89.458) (end 153.404 89.408) (width 0.2032) (layer F.Cu) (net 3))
 (segment (start 153.404 91.39) (end 153.454 91.44) (width 0.2032) (layer F.Cu) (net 3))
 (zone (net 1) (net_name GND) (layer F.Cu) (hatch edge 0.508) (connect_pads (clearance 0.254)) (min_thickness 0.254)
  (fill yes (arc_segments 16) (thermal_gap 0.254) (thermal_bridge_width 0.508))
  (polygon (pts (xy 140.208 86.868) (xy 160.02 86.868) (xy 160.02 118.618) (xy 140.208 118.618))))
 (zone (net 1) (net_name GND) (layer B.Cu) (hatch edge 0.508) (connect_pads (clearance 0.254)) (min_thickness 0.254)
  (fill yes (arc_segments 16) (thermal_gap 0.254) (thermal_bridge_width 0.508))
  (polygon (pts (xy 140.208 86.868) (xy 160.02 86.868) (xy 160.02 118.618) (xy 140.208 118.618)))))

